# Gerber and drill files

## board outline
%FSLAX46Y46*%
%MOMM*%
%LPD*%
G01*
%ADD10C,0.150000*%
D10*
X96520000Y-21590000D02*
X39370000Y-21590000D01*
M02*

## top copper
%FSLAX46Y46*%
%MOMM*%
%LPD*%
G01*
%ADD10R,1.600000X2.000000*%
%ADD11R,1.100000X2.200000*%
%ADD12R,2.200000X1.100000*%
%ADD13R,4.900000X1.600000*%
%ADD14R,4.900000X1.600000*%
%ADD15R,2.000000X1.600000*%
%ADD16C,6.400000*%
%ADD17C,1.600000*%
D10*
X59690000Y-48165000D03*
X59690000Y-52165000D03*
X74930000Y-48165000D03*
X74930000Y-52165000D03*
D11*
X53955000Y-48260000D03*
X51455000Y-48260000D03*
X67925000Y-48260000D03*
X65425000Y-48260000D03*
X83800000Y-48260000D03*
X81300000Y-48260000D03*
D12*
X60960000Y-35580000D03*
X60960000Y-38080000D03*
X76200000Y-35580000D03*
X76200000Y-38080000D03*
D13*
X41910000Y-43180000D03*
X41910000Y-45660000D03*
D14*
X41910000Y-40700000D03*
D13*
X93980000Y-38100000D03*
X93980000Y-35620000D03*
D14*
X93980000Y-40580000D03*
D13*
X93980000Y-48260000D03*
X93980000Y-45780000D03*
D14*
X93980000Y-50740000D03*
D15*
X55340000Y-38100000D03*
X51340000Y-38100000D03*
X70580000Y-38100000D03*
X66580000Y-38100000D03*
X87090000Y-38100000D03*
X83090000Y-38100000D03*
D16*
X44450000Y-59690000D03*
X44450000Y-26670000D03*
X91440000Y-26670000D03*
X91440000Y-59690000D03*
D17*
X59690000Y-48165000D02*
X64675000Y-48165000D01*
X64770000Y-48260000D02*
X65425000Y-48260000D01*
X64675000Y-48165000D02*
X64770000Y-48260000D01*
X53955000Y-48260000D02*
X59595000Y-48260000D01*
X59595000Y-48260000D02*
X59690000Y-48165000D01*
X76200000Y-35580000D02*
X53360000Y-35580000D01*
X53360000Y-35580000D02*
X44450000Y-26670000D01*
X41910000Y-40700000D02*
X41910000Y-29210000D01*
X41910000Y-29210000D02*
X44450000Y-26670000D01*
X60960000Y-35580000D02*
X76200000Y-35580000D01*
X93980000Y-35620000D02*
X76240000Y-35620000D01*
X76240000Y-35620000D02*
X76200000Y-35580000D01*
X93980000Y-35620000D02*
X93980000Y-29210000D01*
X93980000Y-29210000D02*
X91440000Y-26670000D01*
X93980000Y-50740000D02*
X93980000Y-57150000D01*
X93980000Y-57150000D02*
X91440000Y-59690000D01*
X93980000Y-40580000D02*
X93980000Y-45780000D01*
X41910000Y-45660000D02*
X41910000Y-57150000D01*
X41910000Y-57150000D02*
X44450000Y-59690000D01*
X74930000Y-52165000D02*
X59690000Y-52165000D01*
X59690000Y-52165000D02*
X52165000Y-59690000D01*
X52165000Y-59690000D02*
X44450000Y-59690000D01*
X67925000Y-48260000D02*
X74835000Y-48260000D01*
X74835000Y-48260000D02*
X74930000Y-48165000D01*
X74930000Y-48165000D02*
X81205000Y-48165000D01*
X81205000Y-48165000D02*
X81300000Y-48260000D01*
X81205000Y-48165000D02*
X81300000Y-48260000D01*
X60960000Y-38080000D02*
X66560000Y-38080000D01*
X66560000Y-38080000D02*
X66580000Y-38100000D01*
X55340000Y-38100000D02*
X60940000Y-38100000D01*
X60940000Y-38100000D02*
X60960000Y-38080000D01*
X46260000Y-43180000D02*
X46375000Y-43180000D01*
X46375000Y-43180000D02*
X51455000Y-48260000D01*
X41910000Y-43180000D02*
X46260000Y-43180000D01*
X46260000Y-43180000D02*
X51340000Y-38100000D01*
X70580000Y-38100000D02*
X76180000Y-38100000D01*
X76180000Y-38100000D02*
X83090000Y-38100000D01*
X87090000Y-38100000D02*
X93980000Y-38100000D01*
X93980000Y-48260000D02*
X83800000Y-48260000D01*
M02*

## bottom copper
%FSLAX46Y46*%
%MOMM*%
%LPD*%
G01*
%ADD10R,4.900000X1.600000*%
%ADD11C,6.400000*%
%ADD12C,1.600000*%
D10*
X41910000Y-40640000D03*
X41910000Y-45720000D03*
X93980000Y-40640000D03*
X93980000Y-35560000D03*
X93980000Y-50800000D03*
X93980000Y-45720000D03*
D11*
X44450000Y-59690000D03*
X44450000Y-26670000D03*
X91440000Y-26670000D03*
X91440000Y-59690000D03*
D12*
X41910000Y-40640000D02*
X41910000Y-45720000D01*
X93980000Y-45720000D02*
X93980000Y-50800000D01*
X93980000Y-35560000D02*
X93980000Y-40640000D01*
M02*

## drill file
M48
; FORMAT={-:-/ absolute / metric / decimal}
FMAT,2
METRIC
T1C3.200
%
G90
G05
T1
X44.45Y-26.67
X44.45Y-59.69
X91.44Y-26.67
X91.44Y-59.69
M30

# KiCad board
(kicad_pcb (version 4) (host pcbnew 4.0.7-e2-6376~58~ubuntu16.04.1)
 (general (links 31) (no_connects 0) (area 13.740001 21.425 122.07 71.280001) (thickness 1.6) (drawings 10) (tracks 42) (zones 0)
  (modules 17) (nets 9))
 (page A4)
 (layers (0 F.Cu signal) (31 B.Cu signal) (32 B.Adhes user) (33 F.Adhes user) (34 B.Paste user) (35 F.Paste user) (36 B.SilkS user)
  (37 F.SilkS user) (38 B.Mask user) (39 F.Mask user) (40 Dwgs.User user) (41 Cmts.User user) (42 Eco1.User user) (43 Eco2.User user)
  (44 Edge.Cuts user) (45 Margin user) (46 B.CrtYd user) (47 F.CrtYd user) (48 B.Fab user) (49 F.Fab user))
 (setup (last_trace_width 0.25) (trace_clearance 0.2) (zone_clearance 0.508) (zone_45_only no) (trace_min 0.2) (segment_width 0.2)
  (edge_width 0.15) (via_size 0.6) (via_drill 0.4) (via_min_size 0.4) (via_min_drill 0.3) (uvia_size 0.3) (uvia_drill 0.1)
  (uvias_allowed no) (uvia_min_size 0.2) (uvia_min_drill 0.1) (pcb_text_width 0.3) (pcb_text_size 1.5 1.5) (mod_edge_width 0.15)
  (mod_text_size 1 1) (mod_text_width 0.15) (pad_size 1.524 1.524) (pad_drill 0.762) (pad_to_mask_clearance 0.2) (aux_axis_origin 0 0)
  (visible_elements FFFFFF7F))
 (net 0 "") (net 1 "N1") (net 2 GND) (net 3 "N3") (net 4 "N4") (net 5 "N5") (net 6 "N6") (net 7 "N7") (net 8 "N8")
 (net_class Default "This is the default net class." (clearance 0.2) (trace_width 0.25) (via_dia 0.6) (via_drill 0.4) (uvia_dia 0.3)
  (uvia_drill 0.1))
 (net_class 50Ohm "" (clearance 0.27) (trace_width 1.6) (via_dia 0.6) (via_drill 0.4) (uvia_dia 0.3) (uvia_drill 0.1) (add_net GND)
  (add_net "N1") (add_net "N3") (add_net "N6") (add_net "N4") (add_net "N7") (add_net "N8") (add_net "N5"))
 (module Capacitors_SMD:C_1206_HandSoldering (layer F.Cu) (at 59.69 50.165 270)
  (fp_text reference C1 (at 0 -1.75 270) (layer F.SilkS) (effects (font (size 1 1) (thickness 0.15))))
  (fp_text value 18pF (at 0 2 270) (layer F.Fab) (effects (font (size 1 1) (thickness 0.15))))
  (pad 1 smd rect (at -2 0 270) (size 2 1.6) (layers F.Cu F.Paste F.Mask) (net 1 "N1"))
  (pad 2 smd rect (at 2 0 270) (size 2 1.6) (layers F.Cu F.Paste F.Mask) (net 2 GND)))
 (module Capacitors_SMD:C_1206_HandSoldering (layer F.Cu) (at 74.93 50.165 270)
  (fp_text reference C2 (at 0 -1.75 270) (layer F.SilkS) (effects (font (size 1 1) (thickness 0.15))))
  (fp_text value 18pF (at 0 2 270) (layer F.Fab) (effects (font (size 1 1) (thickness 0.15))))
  (pad 1 smd rect (at -2 0 270) (size 2 1.6) (layers F.Cu F.Paste F.Mask) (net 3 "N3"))
  (pad 2 smd rect (at 2 0 270) (size 2 1.6) (layers F.Cu F.Paste F.Mask) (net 2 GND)))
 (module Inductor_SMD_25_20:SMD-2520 (layer F.Cu) (at 52.705 48.26 270)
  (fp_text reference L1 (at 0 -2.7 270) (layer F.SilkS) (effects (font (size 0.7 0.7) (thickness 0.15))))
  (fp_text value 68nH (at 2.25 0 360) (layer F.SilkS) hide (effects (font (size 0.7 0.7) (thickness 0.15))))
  (pad 1 smd rect (at 0 -1.25 270) (size 2.2 1.1) (layers F.Cu F.Paste F.Mask) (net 1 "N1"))
  (pad 2 smd rect (at 0 1.25 270) (size 2.2 1.1) (layers F.Cu F.Paste F.Mask) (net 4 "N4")))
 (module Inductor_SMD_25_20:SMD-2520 (layer F.Cu) (at 66.675 48.26 270)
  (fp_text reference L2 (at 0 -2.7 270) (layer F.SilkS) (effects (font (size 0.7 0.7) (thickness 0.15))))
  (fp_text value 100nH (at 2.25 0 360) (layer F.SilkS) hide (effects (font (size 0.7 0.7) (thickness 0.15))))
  (pad 1 smd rect (at 0 -1.25 270) (size 2.2 1.1) (layers F.Cu F.Paste F.Mask) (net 3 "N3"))
  (pad 2 smd rect (at 0 1.25 270) (size 2.2 1.1) (layers F.Cu F.Paste F.Mask) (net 1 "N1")))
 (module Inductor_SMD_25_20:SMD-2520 (layer F.Cu) (at 82.55 48.26 270)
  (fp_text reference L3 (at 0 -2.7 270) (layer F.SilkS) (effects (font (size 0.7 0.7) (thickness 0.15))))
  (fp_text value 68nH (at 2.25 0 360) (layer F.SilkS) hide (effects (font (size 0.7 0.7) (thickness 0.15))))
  (pad 1 smd rect (at 0 -1.25 270) (size 2.2 1.1) (layers F.Cu F.Paste F.Mask) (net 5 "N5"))
  (pad 2 smd rect (at 0 1.25 270) (size 2.2 1.1) (layers F.Cu F.Paste F.Mask) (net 3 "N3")))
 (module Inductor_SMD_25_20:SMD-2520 (layer F.Cu) (at 60.96 36.83)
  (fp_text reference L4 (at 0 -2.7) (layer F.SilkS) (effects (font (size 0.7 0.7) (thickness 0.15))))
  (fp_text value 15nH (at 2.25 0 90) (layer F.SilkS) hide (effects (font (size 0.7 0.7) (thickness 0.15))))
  (pad 1 smd rect (at 0 -1.25) (size 2.2 1.1) (layers F.Cu F.Paste F.Mask) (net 2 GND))
  (pad 2 smd rect (at 0 1.25) (size 2.2 1.1) (layers F.Cu F.Paste F.Mask) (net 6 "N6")))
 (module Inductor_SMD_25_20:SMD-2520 (layer F.Cu) (at 76.2 36.83)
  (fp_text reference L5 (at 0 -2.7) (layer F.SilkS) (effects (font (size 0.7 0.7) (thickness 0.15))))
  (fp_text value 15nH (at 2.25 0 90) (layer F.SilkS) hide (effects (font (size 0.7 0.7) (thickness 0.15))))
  (pad 1 smd rect (at 0 -1.25) (size 2.2 1.1) (layers F.Cu F.Paste F.Mask) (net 2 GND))
  (pad 2 smd rect (at 0 1.25) (size 2.2 1.1) (layers F.Cu F.Paste F.Mask) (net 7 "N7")))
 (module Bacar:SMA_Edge (layer F.Cu) (at 41.91 43.18 90)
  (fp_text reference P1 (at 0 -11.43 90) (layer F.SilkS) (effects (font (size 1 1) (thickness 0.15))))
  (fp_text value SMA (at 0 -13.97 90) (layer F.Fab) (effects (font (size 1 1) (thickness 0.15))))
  (pad 1 connect rect (at 0 0 90) (size 1.6 4.9) (layers F.Cu F.Mask) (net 4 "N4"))
  (pad 2 connect rect (at -2.48 0 90) (size 1.6 4.9) (layers F.Cu F.Mask) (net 2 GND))
  (pad 2 smd rect (at 2.48 0 90) (size 1.6 4.9) (layers F.Cu F.Paste F.Mask) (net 2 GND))
  (pad 2 smd rect (at 2.54 0 90) (size 1.6 4.9) (layers B.Cu F.Paste F.Mask) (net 2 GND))
  (pad 2 smd rect (at -2.54 0 90) (size 1.6 4.9) (layers B.Cu F.Paste F.Mask) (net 2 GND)))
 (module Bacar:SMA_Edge (layer F.Cu) (at 93.98 38.1 270)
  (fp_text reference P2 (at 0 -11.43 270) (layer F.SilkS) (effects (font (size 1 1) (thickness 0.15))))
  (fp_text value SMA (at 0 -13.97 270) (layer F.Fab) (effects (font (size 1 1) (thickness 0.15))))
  (pad 1 connect rect (at 0 0 270) (size 1.6 4.9) (layers F.Cu F.Mask) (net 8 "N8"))
  (pad 2 connect rect (at -2.48 0 270) (size 1.6 4.9) (layers F.Cu F.Mask) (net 2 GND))
  (pad 2 smd rect (at 2.48 0 270) (size 1.6 4.9) (layers F.Cu F.Paste F.Mask) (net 2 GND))
  (pad 2 smd rect (at 2.54 0 270) (size 1.6 4.9) (layers B.Cu F.Paste F.Mask) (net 2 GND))
  (pad 2 smd rect (at -2.54 0 270) (size 1.6 4.9) (layers B.Cu F.Paste F.Mask) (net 2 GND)))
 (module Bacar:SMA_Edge (layer F.Cu) (at 93.98 48.26 270)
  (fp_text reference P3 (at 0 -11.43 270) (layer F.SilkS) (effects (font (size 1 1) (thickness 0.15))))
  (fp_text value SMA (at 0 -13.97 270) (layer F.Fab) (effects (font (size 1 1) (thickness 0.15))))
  (pad 1 connect rect (at 0 0 270) (size 1.6 4.9) (layers F.Cu F.Mask) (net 5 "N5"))
  (pad 2 connect rect (at -2.48 0 270) (size 1.6 4.9) (layers F.Cu F.Mask) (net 2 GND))
  (pad 2 smd rect (at 2.48 0 270) (size 1.6 4.9) (layers F.Cu F.Paste F.Mask) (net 2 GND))
  (pad 2 smd rect (at 2.54 0 270) (size 1.6 4.9) (layers B.Cu F.Paste F.Mask) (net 2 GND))
  (pad 2 smd rect (at -2.54 0 270) (size 1.6 4.9) (layers B.Cu F.Paste F.Mask) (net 2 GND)))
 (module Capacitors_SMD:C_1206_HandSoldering (layer F.Cu) (at 53.34 38.1 180)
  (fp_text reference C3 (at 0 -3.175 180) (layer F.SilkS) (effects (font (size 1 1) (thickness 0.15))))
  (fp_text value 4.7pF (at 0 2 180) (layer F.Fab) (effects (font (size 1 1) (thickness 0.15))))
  (pad 1 smd rect (at -2 0 180) (size 2 1.6) (layers F.Cu F.Paste F.Mask) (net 6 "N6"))
  (pad 2 smd rect (at 2 0 180) (size 2 1.6) (layers F.Cu F.Paste F.Mask) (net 4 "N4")))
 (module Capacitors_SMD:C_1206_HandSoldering (layer F.Cu) (at 68.58 38.1 180)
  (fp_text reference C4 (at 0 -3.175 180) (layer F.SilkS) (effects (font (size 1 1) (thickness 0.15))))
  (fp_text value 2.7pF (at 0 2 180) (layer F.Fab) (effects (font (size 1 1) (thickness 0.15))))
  (pad 1 smd rect (at -2 0 180) (size 2 1.6) (layers F.Cu F.Paste F.Mask) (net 7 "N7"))
  (pad 2 smd rect (at 2 0 180) (size 2 1.6) (layers F.Cu F.Paste F.Mask) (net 6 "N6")))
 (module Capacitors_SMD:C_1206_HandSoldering (layer F.Cu) (at 85.09 38.1 180)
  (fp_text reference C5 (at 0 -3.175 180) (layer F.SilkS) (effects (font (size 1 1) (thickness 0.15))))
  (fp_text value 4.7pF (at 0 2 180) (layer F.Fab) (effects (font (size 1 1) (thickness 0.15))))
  (pad 1 smd rect (at -2 0 180) (size 2 1.6) (layers F.Cu F.Paste F.Mask) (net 8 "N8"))
  (pad 2 smd rect (at 2 0 180) (size 2 1.6) (layers F.Cu F.Paste F.Mask) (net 7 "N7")))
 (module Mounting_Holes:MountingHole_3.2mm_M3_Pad (layer F.Cu) (at 44.45 59.69)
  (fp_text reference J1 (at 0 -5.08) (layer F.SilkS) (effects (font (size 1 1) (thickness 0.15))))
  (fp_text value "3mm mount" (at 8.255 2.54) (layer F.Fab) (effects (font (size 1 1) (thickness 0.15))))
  (pad 1 thru_hole circle (at 0 0) (size 6.4 6.4) (drill 3.2) (layers *.Cu *.Mask) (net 2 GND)))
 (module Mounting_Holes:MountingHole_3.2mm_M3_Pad (layer F.Cu) (at 44.45 26.67)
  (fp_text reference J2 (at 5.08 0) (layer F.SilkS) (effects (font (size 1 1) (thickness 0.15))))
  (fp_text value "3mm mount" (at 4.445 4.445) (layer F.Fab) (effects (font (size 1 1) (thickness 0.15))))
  (pad 1 thru_hole circle (at 0 0) (size 6.4 6.4) (drill 3.2) (layers *.Cu *.Mask) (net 2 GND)))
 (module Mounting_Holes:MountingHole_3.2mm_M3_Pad (layer F.Cu) (at 91.44 26.67)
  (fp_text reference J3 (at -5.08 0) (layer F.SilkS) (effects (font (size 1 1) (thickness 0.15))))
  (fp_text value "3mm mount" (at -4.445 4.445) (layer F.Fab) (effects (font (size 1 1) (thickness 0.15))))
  (pad 1 thru_hole circle (at 0 0) (size 6.4 6.4) (drill 3.2) (layers *.Cu *.Mask) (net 2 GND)))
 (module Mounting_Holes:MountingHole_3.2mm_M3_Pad (layer F.Cu) (at 91.44 59.69)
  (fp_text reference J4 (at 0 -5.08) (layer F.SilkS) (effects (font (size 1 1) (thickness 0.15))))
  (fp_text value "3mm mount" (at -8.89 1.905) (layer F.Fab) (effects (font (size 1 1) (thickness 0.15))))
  (pad 1 thru_hole circle (at 0 0) (size 6.4 6.4) (drill 3.2) (layers *.Cu *.Mask) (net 2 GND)))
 (gr_line (start 96.52 21.59) (end 39.37 21.59) (angle 90) (layer Edge.Cuts) (width 0.15))
 (segment (start 59.69 48.165) (end 64.675 48.165) (width 1.6) (layer F.Cu) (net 1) (status 400000))
 (segment (start 64.77 48.26) (end 65.425 48.26) (width 1.6) (layer F.Cu) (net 1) (status 800000))
 (segment (start 64.675 48.165) (end 64.77 48.26) (width 1.6) (layer F.Cu) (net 1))
 (segment (start 53.955 48.26) (end 59.595 48.26) (width 1.6) (layer F.Cu) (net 1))
 (segment (start 59.595 48.26) (end 59.69 48.165) (width 1.6) (layer F.Cu) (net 1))
 (segment (start 76.2 35.58) (end 53.36 35.58) (width 1.6) (layer F.Cu) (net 2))
 (segment (start 53.36 35.58) (end 44.45 26.67) (width 1.6) (layer F.Cu) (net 2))
 (segment (start 41.91 40.7) (end 41.91 29.21) (width 1.6) (layer F.Cu) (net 2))
 (segment (start 41.91 29.21) (end 44.45 26.67) (width 1.6) (layer F.Cu) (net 2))
 (segment (start 41.91 40.64) (end 41.91 45.72) (width 1.6) (layer B.Cu) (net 2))
 (segment (start 93.98 45.72) (end 93.98 50.8) (width 1.6) (layer B.Cu) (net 2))
 (segment (start 93.98 35.56) (end 93.98 40.64) (width 1.6) (layer B.Cu) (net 2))
 (segment (start 60.96 35.58) (end 76.2 35.58) (width 1.6) (layer F.Cu) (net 2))
 (segment (start 93.98 35.62) (end 76.24 35.62) (width 1.6) (layer F.Cu) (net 2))
 (segment (start 76.24 35.62) (end 76.2 35.58) (width 1.6) (layer F.Cu) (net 2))
 (segment (start 93.98 35.62) (end 93.98 29.21) (width 1.6) (layer F.Cu) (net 2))
 (segment (start 93.98 29.21) (end 91.44 26.67) (width 1.6) (layer F.Cu) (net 2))
 (segment (start 93.98 50.74) (end 93.98 57.15) (width 1.6) (layer F.Cu) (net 2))
 (segment (start 93.98 57.15) (end 91.44 59.69) (width 1.6) (layer F.Cu) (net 2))
 (segment (start 93.98 40.58) (end 93.98 45.78) (width 1.6) (layer F.Cu) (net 2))
 (segment (start 41.91 45.66) (end 41.91 57.15) (width 1.6) (layer F.Cu) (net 2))
 (segment (start 41.91 57.15) (end 44.45 59.69) (width 1.6) (layer F.Cu) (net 2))
 (segment (start 74.93 52.165) (end 59.69 52.165) (width 1.6) (layer F.Cu) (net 2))
 (segment (start 59.69 52.165) (end 52.165 59.69) (width 1.6) (layer F.Cu) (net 2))
 (segment (start 52.165 59.69) (end 44.45 59.69) (width 1.6) (layer F.Cu) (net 2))
 (segment (start 67.925 48.26) (end 74.835 48.26) (width 1.6) (layer F.Cu) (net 3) (status C00000))
 (segment (start 74.835 48.26) (end 74.93 48.165) (width 1.6) (layer F.Cu) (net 3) (status C00000))
 (segment (start 74.93 48.165) (end 81.205 48.165) (width 1.6) (layer F.Cu) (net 3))
 (segment (start 81.205 48.165) (end 81.3 48.26) (width 1.6) (layer F.Cu) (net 3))
 (segment (start 81.205 48.165) (end 81.3 48.26) (width 1.6) (layer F.Cu) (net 3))
 (segment (start 60.96 38.08) (end 66.56 38.08) (width 1.6) (layer F.Cu) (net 6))
 (segment (start 66.56 38.08) (end 66.58 38.1) (width 1.6) (layer F.Cu) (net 6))
 (segment (start 55.34 38.1) (end 60.94 38.1) (width 1.6) (layer F.Cu) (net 6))
 (segment (start 60.94 38.1) (end 60.96 38.08) (width 1.6) (layer F.Cu) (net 6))
 (segment (start 46.26 43.18) (end 46.375 43.18) (width 1.6) (layer F.Cu) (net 4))
 (segment (start 46.375 43.18) (end 51.455 48.26) (width 1.6) (layer F.Cu) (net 4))
 (segment (start 41.91 43.18) (end 46.26 43.18) (width 1.6) (layer F.Cu) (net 4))
 (segment (start 46.26 43.18) (end 51.34 38.1) (width 1.6) (layer F.Cu) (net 4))
 (segment (start 70.58 38.1) (end 76.18 38.1) (width 1.6) (layer F.Cu) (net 7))
 (segment (start 76.18 38.1) (end 83.09 38.1) (width 1.6) (layer F.Cu) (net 7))
 (segment (start 87.09 38.1) (end 93.98 38.1) (width 1.6) (layer F.Cu) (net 8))
 (segment (start 93.98 48.26) (end 83.8 48.26) (width 1.6) (layer F.Cu) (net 5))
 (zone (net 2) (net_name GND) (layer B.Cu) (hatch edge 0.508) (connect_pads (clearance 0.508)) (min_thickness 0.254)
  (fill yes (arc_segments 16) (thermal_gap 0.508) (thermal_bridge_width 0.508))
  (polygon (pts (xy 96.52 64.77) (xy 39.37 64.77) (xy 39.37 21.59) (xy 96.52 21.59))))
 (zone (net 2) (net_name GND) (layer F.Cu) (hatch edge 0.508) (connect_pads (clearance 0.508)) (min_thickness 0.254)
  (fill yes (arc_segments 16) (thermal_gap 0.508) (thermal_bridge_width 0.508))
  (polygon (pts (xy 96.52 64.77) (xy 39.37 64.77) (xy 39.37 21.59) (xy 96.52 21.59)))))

